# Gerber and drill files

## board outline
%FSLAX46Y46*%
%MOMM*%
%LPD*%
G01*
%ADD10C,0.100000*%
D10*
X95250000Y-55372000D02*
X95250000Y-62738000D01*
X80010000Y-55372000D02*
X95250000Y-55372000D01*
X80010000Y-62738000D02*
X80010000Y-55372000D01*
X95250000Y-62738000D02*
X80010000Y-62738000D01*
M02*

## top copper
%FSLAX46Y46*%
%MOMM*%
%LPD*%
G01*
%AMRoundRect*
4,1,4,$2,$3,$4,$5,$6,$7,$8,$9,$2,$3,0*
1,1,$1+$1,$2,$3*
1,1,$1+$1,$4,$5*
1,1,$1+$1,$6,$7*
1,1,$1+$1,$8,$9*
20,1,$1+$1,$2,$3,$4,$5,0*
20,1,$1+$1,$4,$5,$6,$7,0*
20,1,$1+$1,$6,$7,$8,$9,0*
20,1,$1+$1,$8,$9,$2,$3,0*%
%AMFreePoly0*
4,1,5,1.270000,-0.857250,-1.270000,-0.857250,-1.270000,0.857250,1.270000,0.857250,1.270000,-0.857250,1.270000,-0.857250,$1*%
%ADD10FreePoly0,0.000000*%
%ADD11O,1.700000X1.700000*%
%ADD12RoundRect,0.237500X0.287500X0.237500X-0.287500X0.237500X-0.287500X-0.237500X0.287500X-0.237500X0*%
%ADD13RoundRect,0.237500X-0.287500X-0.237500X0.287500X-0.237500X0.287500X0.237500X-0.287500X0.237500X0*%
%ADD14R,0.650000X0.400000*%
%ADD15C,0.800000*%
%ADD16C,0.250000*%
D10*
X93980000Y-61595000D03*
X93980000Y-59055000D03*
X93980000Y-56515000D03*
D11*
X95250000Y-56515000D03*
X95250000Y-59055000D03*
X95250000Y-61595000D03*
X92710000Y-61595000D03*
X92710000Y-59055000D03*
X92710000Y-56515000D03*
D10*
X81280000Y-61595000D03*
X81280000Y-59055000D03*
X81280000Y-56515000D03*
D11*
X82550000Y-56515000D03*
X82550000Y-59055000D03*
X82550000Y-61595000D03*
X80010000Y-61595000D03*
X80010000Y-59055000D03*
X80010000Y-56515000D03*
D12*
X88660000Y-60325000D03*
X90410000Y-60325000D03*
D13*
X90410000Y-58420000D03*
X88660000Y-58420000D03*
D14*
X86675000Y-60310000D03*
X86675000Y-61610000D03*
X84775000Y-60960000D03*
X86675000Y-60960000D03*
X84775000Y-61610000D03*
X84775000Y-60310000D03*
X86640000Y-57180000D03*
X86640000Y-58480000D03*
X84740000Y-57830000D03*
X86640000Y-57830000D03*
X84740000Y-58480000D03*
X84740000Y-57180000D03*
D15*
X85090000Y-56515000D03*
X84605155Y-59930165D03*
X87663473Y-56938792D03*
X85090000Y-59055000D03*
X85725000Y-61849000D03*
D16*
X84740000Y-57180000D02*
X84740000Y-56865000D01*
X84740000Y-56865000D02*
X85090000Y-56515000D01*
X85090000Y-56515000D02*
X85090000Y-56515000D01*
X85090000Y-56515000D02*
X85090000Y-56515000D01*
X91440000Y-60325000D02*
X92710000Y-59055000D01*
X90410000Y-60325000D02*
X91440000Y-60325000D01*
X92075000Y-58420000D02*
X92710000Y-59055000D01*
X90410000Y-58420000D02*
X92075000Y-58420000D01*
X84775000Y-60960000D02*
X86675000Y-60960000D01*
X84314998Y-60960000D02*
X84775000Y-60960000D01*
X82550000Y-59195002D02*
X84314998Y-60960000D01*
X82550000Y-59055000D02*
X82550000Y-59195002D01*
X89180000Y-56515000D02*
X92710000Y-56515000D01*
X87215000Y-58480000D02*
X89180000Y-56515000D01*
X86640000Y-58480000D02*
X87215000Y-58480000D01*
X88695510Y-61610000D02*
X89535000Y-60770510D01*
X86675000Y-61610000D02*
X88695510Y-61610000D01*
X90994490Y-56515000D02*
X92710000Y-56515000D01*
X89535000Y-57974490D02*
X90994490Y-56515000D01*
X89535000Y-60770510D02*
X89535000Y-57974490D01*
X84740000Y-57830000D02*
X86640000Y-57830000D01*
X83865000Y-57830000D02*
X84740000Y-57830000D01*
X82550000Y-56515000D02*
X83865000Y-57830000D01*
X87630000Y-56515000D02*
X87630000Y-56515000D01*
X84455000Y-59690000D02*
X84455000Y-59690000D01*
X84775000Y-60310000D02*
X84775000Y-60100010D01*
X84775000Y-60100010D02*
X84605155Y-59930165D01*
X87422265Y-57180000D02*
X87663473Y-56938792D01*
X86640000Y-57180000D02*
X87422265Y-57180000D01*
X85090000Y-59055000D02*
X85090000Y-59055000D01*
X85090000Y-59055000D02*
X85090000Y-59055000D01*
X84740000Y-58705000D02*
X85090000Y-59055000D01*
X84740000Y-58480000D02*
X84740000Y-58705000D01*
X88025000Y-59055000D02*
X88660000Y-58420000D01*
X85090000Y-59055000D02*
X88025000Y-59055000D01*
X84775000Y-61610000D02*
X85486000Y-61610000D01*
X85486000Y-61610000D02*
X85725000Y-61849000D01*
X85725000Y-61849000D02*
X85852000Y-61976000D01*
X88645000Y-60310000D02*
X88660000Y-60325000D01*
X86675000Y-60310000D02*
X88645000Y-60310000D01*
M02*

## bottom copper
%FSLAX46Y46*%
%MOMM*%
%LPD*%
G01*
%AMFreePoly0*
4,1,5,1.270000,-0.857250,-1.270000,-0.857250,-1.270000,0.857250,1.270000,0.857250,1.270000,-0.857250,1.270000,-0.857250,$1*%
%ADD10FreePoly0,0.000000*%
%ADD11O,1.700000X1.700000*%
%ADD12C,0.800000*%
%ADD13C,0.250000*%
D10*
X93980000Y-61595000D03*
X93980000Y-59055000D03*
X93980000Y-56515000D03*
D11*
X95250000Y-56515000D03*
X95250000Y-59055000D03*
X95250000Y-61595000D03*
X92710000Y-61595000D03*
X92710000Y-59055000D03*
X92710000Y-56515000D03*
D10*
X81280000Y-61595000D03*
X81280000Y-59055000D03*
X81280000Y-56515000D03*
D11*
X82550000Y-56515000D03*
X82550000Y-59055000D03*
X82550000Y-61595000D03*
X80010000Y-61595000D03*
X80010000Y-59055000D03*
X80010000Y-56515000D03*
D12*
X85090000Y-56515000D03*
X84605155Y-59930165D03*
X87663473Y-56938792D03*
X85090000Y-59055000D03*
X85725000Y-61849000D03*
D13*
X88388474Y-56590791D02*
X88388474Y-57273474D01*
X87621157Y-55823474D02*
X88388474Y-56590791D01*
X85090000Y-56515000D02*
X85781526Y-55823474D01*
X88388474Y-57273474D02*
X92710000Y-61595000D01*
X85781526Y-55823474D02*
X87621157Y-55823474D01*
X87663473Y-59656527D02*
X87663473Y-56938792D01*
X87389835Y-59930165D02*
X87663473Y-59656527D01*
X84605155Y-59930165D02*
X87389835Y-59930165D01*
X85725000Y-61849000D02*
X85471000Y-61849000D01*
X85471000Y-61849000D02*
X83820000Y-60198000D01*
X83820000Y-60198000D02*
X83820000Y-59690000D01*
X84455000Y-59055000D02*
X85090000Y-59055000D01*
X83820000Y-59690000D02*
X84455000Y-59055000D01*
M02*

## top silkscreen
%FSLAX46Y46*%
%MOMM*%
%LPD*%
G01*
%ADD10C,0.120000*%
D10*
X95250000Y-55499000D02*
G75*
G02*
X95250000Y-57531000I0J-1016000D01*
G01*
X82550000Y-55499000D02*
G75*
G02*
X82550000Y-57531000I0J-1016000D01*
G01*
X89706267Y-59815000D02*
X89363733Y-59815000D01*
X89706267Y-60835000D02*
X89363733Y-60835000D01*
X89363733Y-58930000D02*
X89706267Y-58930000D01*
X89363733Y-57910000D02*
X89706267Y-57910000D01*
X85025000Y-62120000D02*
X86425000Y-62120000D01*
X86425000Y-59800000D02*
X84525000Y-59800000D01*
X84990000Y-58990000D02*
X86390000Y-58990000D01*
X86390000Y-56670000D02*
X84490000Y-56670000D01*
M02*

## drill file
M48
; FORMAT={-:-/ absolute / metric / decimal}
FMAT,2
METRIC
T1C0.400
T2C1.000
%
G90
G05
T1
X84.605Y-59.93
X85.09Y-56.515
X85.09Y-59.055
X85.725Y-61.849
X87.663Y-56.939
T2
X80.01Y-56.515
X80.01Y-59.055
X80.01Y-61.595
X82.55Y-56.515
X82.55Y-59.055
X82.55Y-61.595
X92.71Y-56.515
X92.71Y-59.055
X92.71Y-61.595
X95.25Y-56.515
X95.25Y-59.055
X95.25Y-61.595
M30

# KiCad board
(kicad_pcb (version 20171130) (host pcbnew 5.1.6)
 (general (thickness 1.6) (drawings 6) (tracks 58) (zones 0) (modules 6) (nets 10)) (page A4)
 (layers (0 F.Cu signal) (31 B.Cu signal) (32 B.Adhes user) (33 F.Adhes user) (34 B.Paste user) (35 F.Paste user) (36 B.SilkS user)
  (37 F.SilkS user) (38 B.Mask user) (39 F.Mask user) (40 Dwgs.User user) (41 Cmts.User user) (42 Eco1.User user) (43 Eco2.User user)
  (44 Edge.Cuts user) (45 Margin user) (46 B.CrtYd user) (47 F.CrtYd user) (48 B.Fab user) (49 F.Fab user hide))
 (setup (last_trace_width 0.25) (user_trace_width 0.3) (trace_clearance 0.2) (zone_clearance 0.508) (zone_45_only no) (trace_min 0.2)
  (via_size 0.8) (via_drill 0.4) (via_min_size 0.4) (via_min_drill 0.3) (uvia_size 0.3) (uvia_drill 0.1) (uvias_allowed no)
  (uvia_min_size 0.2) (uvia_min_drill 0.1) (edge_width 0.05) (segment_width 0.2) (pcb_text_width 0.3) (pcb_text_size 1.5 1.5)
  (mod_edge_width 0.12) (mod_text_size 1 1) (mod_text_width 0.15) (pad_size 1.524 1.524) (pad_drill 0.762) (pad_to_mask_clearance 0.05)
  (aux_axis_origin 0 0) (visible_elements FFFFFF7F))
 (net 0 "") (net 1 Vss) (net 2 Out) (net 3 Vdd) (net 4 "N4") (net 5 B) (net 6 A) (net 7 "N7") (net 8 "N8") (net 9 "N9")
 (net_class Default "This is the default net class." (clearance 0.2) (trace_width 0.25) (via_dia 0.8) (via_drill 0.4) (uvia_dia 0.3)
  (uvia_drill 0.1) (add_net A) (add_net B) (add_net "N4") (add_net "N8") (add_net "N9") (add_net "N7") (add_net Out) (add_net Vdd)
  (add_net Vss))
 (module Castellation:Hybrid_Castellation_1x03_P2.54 (layer F.Cu) (at 93.98 56.515)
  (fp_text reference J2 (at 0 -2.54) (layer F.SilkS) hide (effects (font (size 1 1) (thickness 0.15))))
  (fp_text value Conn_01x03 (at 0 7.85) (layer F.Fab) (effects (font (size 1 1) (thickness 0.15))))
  (fp_arc (start 1.27 0) (end 1.27 1.016) (angle -180) (layer F.SilkS) (width 0.12))
  (pad 3 connect custom (at 0 5.08) (size 2.54 1.7145) (layers B.Cu B.Mask) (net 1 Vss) (zone_connect 0)
   (options (clearance outline) (anchor rect)) (primitives))
  (pad 2 connect custom (at 0 2.54) (size 2.54 1.7145) (layers B.Cu B.Mask) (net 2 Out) (zone_connect 0)
   (options (clearance outline) (anchor rect)) (primitives))
  (pad 1 connect custom (at 0 0) (size 2.54 1.7145) (layers B.Cu B.Mask) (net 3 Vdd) (zone_connect 0)
   (options (clearance outline) (anchor rect)) (primitives))
  (pad 3 connect custom (at 0 5.08) (size 2.54 1.7145) (layers F.Cu F.Mask) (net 1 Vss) (zone_connect 0)
   (options (clearance outline) (anchor rect)) (primitives))
  (pad 2 connect custom (at 0 2.54) (size 2.54 1.7145) (layers F.Cu F.Mask) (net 2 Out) (zone_connect 0)
   (options (clearance outline) (anchor rect)) (primitives))
  (pad 1 connect custom (at 0 0) (size 2.54 1.7145) (layers F.Cu F.Mask) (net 3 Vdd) (zone_connect 0)
   (options (clearance outline) (anchor rect)) (primitives))
  (pad 1 thru_hole oval (at 1.27 0) (size 1.7 1.7) (drill 1) (layers *.Cu *.Mask) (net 3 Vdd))
  (pad 2 thru_hole oval (at 1.27 2.54) (size 1.7 1.7) (drill 1) (layers *.Cu *.Mask) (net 2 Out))
  (pad 3 thru_hole oval (at 1.27 5.08) (size 1.7 1.7) (drill 1) (layers *.Cu *.Mask) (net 1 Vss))
  (pad 3 thru_hole oval (at -1.27 5.08) (size 1.7 1.7) (drill 1) (layers *.Cu *.Mask) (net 1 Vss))
  (pad 2 thru_hole oval (at -1.27 2.54) (size 1.7 1.7) (drill 1) (layers *.Cu *.Mask) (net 2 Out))
  (pad 1 thru_hole oval (at -1.27 0) (size 1.7 1.7) (drill 1) (layers *.Cu *.Mask) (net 3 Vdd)))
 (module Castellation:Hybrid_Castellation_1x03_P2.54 (layer F.Cu) (at 81.28 56.515)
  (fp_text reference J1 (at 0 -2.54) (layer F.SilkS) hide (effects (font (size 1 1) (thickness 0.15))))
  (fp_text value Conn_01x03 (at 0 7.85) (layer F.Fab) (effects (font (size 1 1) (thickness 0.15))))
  (fp_arc (start 1.27 0) (end 1.27 1.016) (angle -180) (layer F.SilkS) (width 0.12))
  (pad 3 connect custom (at 0 5.08) (size 2.54 1.7145) (layers B.Cu B.Mask) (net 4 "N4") (zone_connect 0)
   (options (clearance outline) (anchor rect)) (primitives))
  (pad 2 connect custom (at 0 2.54) (size 2.54 1.7145) (layers B.Cu B.Mask) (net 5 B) (zone_connect 0)
   (options (clearance outline) (anchor rect)) (primitives))
  (pad 1 connect custom (at 0 0) (size 2.54 1.7145) (layers B.Cu B.Mask) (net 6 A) (zone_connect 0)
   (options (clearance outline) (anchor rect)) (primitives))
  (pad 3 connect custom (at 0 5.08) (size 2.54 1.7145) (layers F.Cu F.Mask) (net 4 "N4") (zone_connect 0)
   (options (clearance outline) (anchor rect)) (primitives))
  (pad 2 connect custom (at 0 2.54) (size 2.54 1.7145) (layers F.Cu F.Mask) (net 5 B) (zone_connect 0)
   (options (clearance outline) (anchor rect)) (primitives))
  (pad 1 connect custom (at 0 0) (size 2.54 1.7145) (layers F.Cu F.Mask) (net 6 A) (zone_connect 0)
   (options (clearance outline) (anchor rect)) (primitives))
  (pad 1 thru_hole oval (at 1.27 0) (size 1.7 1.7) (drill 1) (layers *.Cu *.Mask) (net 6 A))
  (pad 2 thru_hole oval (at 1.27 2.54) (size 1.7 1.7) (drill 1) (layers *.Cu *.Mask) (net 5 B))
  (pad 3 thru_hole oval (at 1.27 5.08) (size 1.7 1.7) (drill 1) (layers *.Cu *.Mask) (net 4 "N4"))
  (pad 3 thru_hole oval (at -1.27 5.08) (size 1.7 1.7) (drill 1) (layers *.Cu *.Mask) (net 4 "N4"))
  (pad 2 thru_hole oval (at -1.27 2.54) (size 1.7 1.7) (drill 1) (layers *.Cu *.Mask) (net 5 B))
  (pad 1 thru_hole oval (at -1.27 0) (size 1.7 1.7) (drill 1) (layers *.Cu *.Mask) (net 6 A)))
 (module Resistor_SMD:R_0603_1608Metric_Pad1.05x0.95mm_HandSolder (layer F.Cu) (at 89.535 60.325 180)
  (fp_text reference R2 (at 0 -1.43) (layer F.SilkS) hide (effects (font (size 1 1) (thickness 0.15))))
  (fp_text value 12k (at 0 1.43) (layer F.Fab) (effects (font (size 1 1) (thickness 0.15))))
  (fp_line (start -0.171267 0.51) (end 0.171267 0.51) (layer F.SilkS) (width 0.12))
  (fp_line (start -0.171267 -0.51) (end 0.171267 -0.51) (layer F.SilkS) (width 0.12))
  (pad 2 smd roundrect (at 0.875 0 180) (size 1.05 0.95) (layers F.Cu F.Paste F.Mask) (roundrect_rratio 0.25) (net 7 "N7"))
  (pad 1 smd roundrect (at -0.875 0 180) (size 1.05 0.95) (layers F.Cu F.Paste F.Mask) (roundrect_rratio 0.25) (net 2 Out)))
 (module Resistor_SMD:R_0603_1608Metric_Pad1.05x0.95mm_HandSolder (layer F.Cu) (at 89.535 58.42)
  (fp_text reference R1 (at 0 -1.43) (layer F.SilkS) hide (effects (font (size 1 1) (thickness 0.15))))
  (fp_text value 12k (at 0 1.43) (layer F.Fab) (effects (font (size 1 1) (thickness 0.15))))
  (fp_line (start -0.171267 0.51) (end 0.171267 0.51) (layer F.SilkS) (width 0.12))
  (fp_line (start -0.171267 -0.51) (end 0.171267 -0.51) (layer F.SilkS) (width 0.12))
  (pad 2 smd roundrect (at 0.875 0) (size 1.05 0.95) (layers F.Cu F.Paste F.Mask) (roundrect_rratio 0.25) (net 2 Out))
  (pad 1 smd roundrect (at -0.875 0) (size 1.05 0.95) (layers F.Cu F.Paste F.Mask) (roundrect_rratio 0.25) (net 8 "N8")))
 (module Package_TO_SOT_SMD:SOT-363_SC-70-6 (layer F.Cu) (at 85.725 60.96)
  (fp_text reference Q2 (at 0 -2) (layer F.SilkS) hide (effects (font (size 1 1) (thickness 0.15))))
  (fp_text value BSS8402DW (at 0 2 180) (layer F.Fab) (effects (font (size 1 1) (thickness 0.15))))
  (fp_line (start -0.7 1.16) (end 0.7 1.16) (layer F.SilkS) (width 0.12))
  (fp_line (start 0.7 -1.16) (end -1.2 -1.16) (layer F.SilkS) (width 0.12))
  (pad 6 smd rect (at 0.95 -0.65) (size 0.65 0.4) (layers F.Cu F.Paste F.Mask) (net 7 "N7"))
  (pad 4 smd rect (at 0.95 0.65) (size 0.65 0.4) (layers F.Cu F.Paste F.Mask) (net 3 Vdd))
  (pad 2 smd rect (at -0.95 0) (size 0.65 0.4) (layers F.Cu F.Paste F.Mask) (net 5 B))
  (pad 5 smd rect (at 0.95 0) (size 0.65 0.4) (layers F.Cu F.Paste F.Mask) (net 5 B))
  (pad 3 smd rect (at -0.95 0.65) (size 0.65 0.4) (layers F.Cu F.Paste F.Mask) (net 8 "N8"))
  (pad 1 smd rect (at -0.95 -0.65) (size 0.65 0.4) (layers F.Cu F.Paste F.Mask) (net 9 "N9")))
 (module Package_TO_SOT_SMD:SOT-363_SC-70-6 (layer F.Cu) (at 85.69 57.83)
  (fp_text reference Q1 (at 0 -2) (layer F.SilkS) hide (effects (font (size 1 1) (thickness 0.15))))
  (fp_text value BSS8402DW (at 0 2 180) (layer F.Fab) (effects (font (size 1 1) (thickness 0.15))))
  (fp_line (start -0.7 1.16) (end 0.7 1.16) (layer F.SilkS) (width 0.12))
  (fp_line (start 0.7 -1.16) (end -1.2 -1.16) (layer F.SilkS) (width 0.12))
  (pad 6 smd rect (at 0.95 -0.65) (size 0.65 0.4) (layers F.Cu F.Paste F.Mask) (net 9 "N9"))
  (pad 4 smd rect (at 0.95 0.65) (size 0.65 0.4) (layers F.Cu F.Paste F.Mask) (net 3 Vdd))
  (pad 2 smd rect (at -0.95 0) (size 0.65 0.4) (layers F.Cu F.Paste F.Mask) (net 6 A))
  (pad 5 smd rect (at 0.95 0) (size 0.65 0.4) (layers F.Cu F.Paste F.Mask) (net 6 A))
  (pad 3 smd rect (at -0.95 0.65) (size 0.65 0.4) (layers F.Cu F.Paste F.Mask) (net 8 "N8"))
  (pad 1 smd rect (at -0.95 -0.65) (size 0.65 0.4) (layers F.Cu F.Paste F.Mask) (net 1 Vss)))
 (gr_line (start 95.25 55.372) (end 95.25 62.738) (layer Edge.Cuts) (width 0.1))
 (gr_line (start 80.01 55.372) (end 95.25 55.372) (layer Edge.Cuts) (width 0.1))
 (gr_line (start 80.01 62.738) (end 80.01 55.372) (layer Edge.Cuts) (width 0.1))
 (gr_line (start 95.25 62.738) (end 80.01 62.738) (layer Edge.Cuts) (width 0.1))
 (segment (start 84.74 57.18) (end 84.74 56.865) (width 0.25) (layer F.Cu) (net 1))
 (segment (start 84.74 56.865) (end 85.09 56.515) (width 0.25) (layer F.Cu) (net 1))
 (segment (start 85.09 56.515) (end 85.09 56.515) (width 0.25) (layer F.Cu) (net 1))
 (segment (start 85.09 56.515) (end 85.09 56.515) (width 0.25) (layer F.Cu) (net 1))
 (via (at 85.09 56.515) (size 0.8) (drill 0.4) (layers F.Cu B.Cu) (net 1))
 (segment (start 88.388474 56.590791) (end 88.388474 57.273474) (width 0.25) (layer B.Cu) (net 1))
 (segment (start 87.621157 55.823474) (end 88.388474 56.590791) (width 0.25) (layer B.Cu) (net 1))
 (segment (start 85.09 56.515) (end 85.781526 55.823474) (width 0.25) (layer B.Cu) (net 1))
 (segment (start 88.388474 57.273474) (end 92.71 61.595) (width 0.25) (layer B.Cu) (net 1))
 (segment (start 85.781526 55.823474) (end 87.621157 55.823474) (width 0.25) (layer B.Cu) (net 1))
 (segment (start 91.44 60.325) (end 92.71 59.055) (width 0.25) (layer F.Cu) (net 2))
 (segment (start 90.41 60.325) (end 91.44 60.325) (width 0.25) (layer F.Cu) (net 2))
 (segment (start 92.075 58.42) (end 92.71 59.055) (width 0.25) (layer F.Cu) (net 2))
 (segment (start 90.41 58.42) (end 92.075 58.42) (width 0.25) (layer F.Cu) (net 2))
 (segment (start 84.775 60.96) (end 86.675 60.96) (width 0.25) (layer F.Cu) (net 5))
 (segment (start 84.314998 60.96) (end 84.775 60.96) (width 0.25) (layer F.Cu) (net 5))
 (segment (start 82.55 59.195002) (end 84.314998 60.96) (width 0.25) (layer F.Cu) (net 5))
 (segment (start 82.55 59.055) (end 82.55 59.195002) (width 0.25) (layer F.Cu) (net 5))
 (segment (start 89.18 56.515) (end 92.71 56.515) (width 0.25) (layer F.Cu) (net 3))
 (segment (start 87.215 58.48) (end 89.18 56.515) (width 0.25) (layer F.Cu) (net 3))
 (segment (start 86.64 58.48) (end 87.215 58.48) (width 0.25) (layer F.Cu) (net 3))
 (segment (start 88.69551 61.61) (end 89.535 60.77051) (width 0.25) (layer F.Cu) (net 3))
 (segment (start 86.675 61.61) (end 88.69551 61.61) (width 0.25) (layer F.Cu) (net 3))
 (segment (start 90.99449 56.515) (end 92.71 56.515) (width 0.25) (layer F.Cu) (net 3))
 (segment (start 89.535 57.97449) (end 90.99449 56.515) (width 0.25) (layer F.Cu) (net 3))
 (segment (start 89.535 60.77051) (end 89.535 57.97449) (width 0.25) (layer F.Cu) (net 3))
 (segment (start 84.74 57.83) (end 86.64 57.83) (width 0.25) (layer F.Cu) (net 6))
 (segment (start 83.865 57.83) (end 84.74 57.83) (width 0.25) (layer F.Cu) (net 6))
 (segment (start 82.55 56.515) (end 83.865 57.83) (width 0.25) (layer F.Cu) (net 6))
 (segment (start 87.63 56.515) (end 87.63 56.515) (width 0.25) (layer F.Cu) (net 9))
 (segment (start 84.455 59.69) (end 84.455 59.69) (width 0.25) (layer F.Cu) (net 9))
 (segment (start 84.775 60.31) (end 84.775 60.10001) (width 0.25) (layer F.Cu) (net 9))
 (segment (start 84.775 60.10001) (end 84.605155 59.930165) (width 0.25) (layer F.Cu) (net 9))
 (via (at 84.605155 59.930165) (size 0.8) (drill 0.4) (layers F.Cu B.Cu) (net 9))
 (segment (start 87.663473 59.656527) (end 87.663473 56.938792) (width 0.25) (layer B.Cu) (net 9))
 (segment (start 87.422265 57.18) (end 87.663473 56.938792) (width 0.25) (layer F.Cu) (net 9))
 (via (at 87.663473 56.938792) (size 0.8) (drill 0.4) (layers F.Cu B.Cu) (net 9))
 (segment (start 86.64 57.18) (end 87.422265 57.18) (width 0.25) (layer F.Cu) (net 9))
 (segment (start 87.389835 59.930165) (end 87.663473 59.656527) (width 0.25) (layer B.Cu) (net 9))
 (segment (start 84.605155 59.930165) (end 87.389835 59.930165) (width 0.25) (layer B.Cu) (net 9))
 (segment (start 85.09 59.055) (end 85.09 59.055) (width 0.25) (layer F.Cu) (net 8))
 (segment (start 85.09 59.055) (end 85.09 59.055) (width 0.25) (layer F.Cu) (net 8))
 (segment (start 84.74 58.705) (end 85.09 59.055) (width 0.25) (layer F.Cu) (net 8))
 (segment (start 84.74 58.48) (end 84.74 58.705) (width 0.25) (layer F.Cu) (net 8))
 (segment (start 88.025 59.055) (end 88.66 58.42) (width 0.25) (layer F.Cu) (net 8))
 (via (at 85.09 59.055) (size 0.8) (drill 0.4) (layers F.Cu B.Cu) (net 8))
 (segment (start 85.09 59.055) (end 88.025 59.055) (width 0.25) (layer F.Cu) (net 8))
 (segment (start 84.775 61.61) (end 85.486 61.61) (width 0.25) (layer F.Cu) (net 8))
 (segment (start 85.486 61.61) (end 85.725 61.849) (width 0.25) (layer F.Cu) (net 8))
 (segment (start 85.725 61.849) (end 85.852 61.976) (width 0.25) (layer F.Cu) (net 8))
 (via (at 85.725 61.849) (size 0.8) (drill 0.4) (layers F.Cu B.Cu) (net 8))
 (segment (start 85.725 61.849) (end 85.471 61.849) (width 0.25) (layer B.Cu) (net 8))
 (segment (start 85.471 61.849) (end 83.82 60.198) (width 0.25) (layer B.Cu) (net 8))
 (segment (start 83.82 60.198) (end 83.82 59.69) (width 0.25) (layer B.Cu) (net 8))
 (segment (start 84.455 59.055) (end 85.09 59.055) (width 0.25) (layer B.Cu) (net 8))
 (segment (start 83.82 59.69) (end 84.455 59.055) (width 0.25) (layer B.Cu) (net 8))
 (segment (start 88.645 60.31) (end 88.66 60.325) (width 0.25) (layer F.Cu) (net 7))
 (segment (start 86.675 60.31) (end 88.645 60.31) (width 0.25) (layer F.Cu) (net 7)))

